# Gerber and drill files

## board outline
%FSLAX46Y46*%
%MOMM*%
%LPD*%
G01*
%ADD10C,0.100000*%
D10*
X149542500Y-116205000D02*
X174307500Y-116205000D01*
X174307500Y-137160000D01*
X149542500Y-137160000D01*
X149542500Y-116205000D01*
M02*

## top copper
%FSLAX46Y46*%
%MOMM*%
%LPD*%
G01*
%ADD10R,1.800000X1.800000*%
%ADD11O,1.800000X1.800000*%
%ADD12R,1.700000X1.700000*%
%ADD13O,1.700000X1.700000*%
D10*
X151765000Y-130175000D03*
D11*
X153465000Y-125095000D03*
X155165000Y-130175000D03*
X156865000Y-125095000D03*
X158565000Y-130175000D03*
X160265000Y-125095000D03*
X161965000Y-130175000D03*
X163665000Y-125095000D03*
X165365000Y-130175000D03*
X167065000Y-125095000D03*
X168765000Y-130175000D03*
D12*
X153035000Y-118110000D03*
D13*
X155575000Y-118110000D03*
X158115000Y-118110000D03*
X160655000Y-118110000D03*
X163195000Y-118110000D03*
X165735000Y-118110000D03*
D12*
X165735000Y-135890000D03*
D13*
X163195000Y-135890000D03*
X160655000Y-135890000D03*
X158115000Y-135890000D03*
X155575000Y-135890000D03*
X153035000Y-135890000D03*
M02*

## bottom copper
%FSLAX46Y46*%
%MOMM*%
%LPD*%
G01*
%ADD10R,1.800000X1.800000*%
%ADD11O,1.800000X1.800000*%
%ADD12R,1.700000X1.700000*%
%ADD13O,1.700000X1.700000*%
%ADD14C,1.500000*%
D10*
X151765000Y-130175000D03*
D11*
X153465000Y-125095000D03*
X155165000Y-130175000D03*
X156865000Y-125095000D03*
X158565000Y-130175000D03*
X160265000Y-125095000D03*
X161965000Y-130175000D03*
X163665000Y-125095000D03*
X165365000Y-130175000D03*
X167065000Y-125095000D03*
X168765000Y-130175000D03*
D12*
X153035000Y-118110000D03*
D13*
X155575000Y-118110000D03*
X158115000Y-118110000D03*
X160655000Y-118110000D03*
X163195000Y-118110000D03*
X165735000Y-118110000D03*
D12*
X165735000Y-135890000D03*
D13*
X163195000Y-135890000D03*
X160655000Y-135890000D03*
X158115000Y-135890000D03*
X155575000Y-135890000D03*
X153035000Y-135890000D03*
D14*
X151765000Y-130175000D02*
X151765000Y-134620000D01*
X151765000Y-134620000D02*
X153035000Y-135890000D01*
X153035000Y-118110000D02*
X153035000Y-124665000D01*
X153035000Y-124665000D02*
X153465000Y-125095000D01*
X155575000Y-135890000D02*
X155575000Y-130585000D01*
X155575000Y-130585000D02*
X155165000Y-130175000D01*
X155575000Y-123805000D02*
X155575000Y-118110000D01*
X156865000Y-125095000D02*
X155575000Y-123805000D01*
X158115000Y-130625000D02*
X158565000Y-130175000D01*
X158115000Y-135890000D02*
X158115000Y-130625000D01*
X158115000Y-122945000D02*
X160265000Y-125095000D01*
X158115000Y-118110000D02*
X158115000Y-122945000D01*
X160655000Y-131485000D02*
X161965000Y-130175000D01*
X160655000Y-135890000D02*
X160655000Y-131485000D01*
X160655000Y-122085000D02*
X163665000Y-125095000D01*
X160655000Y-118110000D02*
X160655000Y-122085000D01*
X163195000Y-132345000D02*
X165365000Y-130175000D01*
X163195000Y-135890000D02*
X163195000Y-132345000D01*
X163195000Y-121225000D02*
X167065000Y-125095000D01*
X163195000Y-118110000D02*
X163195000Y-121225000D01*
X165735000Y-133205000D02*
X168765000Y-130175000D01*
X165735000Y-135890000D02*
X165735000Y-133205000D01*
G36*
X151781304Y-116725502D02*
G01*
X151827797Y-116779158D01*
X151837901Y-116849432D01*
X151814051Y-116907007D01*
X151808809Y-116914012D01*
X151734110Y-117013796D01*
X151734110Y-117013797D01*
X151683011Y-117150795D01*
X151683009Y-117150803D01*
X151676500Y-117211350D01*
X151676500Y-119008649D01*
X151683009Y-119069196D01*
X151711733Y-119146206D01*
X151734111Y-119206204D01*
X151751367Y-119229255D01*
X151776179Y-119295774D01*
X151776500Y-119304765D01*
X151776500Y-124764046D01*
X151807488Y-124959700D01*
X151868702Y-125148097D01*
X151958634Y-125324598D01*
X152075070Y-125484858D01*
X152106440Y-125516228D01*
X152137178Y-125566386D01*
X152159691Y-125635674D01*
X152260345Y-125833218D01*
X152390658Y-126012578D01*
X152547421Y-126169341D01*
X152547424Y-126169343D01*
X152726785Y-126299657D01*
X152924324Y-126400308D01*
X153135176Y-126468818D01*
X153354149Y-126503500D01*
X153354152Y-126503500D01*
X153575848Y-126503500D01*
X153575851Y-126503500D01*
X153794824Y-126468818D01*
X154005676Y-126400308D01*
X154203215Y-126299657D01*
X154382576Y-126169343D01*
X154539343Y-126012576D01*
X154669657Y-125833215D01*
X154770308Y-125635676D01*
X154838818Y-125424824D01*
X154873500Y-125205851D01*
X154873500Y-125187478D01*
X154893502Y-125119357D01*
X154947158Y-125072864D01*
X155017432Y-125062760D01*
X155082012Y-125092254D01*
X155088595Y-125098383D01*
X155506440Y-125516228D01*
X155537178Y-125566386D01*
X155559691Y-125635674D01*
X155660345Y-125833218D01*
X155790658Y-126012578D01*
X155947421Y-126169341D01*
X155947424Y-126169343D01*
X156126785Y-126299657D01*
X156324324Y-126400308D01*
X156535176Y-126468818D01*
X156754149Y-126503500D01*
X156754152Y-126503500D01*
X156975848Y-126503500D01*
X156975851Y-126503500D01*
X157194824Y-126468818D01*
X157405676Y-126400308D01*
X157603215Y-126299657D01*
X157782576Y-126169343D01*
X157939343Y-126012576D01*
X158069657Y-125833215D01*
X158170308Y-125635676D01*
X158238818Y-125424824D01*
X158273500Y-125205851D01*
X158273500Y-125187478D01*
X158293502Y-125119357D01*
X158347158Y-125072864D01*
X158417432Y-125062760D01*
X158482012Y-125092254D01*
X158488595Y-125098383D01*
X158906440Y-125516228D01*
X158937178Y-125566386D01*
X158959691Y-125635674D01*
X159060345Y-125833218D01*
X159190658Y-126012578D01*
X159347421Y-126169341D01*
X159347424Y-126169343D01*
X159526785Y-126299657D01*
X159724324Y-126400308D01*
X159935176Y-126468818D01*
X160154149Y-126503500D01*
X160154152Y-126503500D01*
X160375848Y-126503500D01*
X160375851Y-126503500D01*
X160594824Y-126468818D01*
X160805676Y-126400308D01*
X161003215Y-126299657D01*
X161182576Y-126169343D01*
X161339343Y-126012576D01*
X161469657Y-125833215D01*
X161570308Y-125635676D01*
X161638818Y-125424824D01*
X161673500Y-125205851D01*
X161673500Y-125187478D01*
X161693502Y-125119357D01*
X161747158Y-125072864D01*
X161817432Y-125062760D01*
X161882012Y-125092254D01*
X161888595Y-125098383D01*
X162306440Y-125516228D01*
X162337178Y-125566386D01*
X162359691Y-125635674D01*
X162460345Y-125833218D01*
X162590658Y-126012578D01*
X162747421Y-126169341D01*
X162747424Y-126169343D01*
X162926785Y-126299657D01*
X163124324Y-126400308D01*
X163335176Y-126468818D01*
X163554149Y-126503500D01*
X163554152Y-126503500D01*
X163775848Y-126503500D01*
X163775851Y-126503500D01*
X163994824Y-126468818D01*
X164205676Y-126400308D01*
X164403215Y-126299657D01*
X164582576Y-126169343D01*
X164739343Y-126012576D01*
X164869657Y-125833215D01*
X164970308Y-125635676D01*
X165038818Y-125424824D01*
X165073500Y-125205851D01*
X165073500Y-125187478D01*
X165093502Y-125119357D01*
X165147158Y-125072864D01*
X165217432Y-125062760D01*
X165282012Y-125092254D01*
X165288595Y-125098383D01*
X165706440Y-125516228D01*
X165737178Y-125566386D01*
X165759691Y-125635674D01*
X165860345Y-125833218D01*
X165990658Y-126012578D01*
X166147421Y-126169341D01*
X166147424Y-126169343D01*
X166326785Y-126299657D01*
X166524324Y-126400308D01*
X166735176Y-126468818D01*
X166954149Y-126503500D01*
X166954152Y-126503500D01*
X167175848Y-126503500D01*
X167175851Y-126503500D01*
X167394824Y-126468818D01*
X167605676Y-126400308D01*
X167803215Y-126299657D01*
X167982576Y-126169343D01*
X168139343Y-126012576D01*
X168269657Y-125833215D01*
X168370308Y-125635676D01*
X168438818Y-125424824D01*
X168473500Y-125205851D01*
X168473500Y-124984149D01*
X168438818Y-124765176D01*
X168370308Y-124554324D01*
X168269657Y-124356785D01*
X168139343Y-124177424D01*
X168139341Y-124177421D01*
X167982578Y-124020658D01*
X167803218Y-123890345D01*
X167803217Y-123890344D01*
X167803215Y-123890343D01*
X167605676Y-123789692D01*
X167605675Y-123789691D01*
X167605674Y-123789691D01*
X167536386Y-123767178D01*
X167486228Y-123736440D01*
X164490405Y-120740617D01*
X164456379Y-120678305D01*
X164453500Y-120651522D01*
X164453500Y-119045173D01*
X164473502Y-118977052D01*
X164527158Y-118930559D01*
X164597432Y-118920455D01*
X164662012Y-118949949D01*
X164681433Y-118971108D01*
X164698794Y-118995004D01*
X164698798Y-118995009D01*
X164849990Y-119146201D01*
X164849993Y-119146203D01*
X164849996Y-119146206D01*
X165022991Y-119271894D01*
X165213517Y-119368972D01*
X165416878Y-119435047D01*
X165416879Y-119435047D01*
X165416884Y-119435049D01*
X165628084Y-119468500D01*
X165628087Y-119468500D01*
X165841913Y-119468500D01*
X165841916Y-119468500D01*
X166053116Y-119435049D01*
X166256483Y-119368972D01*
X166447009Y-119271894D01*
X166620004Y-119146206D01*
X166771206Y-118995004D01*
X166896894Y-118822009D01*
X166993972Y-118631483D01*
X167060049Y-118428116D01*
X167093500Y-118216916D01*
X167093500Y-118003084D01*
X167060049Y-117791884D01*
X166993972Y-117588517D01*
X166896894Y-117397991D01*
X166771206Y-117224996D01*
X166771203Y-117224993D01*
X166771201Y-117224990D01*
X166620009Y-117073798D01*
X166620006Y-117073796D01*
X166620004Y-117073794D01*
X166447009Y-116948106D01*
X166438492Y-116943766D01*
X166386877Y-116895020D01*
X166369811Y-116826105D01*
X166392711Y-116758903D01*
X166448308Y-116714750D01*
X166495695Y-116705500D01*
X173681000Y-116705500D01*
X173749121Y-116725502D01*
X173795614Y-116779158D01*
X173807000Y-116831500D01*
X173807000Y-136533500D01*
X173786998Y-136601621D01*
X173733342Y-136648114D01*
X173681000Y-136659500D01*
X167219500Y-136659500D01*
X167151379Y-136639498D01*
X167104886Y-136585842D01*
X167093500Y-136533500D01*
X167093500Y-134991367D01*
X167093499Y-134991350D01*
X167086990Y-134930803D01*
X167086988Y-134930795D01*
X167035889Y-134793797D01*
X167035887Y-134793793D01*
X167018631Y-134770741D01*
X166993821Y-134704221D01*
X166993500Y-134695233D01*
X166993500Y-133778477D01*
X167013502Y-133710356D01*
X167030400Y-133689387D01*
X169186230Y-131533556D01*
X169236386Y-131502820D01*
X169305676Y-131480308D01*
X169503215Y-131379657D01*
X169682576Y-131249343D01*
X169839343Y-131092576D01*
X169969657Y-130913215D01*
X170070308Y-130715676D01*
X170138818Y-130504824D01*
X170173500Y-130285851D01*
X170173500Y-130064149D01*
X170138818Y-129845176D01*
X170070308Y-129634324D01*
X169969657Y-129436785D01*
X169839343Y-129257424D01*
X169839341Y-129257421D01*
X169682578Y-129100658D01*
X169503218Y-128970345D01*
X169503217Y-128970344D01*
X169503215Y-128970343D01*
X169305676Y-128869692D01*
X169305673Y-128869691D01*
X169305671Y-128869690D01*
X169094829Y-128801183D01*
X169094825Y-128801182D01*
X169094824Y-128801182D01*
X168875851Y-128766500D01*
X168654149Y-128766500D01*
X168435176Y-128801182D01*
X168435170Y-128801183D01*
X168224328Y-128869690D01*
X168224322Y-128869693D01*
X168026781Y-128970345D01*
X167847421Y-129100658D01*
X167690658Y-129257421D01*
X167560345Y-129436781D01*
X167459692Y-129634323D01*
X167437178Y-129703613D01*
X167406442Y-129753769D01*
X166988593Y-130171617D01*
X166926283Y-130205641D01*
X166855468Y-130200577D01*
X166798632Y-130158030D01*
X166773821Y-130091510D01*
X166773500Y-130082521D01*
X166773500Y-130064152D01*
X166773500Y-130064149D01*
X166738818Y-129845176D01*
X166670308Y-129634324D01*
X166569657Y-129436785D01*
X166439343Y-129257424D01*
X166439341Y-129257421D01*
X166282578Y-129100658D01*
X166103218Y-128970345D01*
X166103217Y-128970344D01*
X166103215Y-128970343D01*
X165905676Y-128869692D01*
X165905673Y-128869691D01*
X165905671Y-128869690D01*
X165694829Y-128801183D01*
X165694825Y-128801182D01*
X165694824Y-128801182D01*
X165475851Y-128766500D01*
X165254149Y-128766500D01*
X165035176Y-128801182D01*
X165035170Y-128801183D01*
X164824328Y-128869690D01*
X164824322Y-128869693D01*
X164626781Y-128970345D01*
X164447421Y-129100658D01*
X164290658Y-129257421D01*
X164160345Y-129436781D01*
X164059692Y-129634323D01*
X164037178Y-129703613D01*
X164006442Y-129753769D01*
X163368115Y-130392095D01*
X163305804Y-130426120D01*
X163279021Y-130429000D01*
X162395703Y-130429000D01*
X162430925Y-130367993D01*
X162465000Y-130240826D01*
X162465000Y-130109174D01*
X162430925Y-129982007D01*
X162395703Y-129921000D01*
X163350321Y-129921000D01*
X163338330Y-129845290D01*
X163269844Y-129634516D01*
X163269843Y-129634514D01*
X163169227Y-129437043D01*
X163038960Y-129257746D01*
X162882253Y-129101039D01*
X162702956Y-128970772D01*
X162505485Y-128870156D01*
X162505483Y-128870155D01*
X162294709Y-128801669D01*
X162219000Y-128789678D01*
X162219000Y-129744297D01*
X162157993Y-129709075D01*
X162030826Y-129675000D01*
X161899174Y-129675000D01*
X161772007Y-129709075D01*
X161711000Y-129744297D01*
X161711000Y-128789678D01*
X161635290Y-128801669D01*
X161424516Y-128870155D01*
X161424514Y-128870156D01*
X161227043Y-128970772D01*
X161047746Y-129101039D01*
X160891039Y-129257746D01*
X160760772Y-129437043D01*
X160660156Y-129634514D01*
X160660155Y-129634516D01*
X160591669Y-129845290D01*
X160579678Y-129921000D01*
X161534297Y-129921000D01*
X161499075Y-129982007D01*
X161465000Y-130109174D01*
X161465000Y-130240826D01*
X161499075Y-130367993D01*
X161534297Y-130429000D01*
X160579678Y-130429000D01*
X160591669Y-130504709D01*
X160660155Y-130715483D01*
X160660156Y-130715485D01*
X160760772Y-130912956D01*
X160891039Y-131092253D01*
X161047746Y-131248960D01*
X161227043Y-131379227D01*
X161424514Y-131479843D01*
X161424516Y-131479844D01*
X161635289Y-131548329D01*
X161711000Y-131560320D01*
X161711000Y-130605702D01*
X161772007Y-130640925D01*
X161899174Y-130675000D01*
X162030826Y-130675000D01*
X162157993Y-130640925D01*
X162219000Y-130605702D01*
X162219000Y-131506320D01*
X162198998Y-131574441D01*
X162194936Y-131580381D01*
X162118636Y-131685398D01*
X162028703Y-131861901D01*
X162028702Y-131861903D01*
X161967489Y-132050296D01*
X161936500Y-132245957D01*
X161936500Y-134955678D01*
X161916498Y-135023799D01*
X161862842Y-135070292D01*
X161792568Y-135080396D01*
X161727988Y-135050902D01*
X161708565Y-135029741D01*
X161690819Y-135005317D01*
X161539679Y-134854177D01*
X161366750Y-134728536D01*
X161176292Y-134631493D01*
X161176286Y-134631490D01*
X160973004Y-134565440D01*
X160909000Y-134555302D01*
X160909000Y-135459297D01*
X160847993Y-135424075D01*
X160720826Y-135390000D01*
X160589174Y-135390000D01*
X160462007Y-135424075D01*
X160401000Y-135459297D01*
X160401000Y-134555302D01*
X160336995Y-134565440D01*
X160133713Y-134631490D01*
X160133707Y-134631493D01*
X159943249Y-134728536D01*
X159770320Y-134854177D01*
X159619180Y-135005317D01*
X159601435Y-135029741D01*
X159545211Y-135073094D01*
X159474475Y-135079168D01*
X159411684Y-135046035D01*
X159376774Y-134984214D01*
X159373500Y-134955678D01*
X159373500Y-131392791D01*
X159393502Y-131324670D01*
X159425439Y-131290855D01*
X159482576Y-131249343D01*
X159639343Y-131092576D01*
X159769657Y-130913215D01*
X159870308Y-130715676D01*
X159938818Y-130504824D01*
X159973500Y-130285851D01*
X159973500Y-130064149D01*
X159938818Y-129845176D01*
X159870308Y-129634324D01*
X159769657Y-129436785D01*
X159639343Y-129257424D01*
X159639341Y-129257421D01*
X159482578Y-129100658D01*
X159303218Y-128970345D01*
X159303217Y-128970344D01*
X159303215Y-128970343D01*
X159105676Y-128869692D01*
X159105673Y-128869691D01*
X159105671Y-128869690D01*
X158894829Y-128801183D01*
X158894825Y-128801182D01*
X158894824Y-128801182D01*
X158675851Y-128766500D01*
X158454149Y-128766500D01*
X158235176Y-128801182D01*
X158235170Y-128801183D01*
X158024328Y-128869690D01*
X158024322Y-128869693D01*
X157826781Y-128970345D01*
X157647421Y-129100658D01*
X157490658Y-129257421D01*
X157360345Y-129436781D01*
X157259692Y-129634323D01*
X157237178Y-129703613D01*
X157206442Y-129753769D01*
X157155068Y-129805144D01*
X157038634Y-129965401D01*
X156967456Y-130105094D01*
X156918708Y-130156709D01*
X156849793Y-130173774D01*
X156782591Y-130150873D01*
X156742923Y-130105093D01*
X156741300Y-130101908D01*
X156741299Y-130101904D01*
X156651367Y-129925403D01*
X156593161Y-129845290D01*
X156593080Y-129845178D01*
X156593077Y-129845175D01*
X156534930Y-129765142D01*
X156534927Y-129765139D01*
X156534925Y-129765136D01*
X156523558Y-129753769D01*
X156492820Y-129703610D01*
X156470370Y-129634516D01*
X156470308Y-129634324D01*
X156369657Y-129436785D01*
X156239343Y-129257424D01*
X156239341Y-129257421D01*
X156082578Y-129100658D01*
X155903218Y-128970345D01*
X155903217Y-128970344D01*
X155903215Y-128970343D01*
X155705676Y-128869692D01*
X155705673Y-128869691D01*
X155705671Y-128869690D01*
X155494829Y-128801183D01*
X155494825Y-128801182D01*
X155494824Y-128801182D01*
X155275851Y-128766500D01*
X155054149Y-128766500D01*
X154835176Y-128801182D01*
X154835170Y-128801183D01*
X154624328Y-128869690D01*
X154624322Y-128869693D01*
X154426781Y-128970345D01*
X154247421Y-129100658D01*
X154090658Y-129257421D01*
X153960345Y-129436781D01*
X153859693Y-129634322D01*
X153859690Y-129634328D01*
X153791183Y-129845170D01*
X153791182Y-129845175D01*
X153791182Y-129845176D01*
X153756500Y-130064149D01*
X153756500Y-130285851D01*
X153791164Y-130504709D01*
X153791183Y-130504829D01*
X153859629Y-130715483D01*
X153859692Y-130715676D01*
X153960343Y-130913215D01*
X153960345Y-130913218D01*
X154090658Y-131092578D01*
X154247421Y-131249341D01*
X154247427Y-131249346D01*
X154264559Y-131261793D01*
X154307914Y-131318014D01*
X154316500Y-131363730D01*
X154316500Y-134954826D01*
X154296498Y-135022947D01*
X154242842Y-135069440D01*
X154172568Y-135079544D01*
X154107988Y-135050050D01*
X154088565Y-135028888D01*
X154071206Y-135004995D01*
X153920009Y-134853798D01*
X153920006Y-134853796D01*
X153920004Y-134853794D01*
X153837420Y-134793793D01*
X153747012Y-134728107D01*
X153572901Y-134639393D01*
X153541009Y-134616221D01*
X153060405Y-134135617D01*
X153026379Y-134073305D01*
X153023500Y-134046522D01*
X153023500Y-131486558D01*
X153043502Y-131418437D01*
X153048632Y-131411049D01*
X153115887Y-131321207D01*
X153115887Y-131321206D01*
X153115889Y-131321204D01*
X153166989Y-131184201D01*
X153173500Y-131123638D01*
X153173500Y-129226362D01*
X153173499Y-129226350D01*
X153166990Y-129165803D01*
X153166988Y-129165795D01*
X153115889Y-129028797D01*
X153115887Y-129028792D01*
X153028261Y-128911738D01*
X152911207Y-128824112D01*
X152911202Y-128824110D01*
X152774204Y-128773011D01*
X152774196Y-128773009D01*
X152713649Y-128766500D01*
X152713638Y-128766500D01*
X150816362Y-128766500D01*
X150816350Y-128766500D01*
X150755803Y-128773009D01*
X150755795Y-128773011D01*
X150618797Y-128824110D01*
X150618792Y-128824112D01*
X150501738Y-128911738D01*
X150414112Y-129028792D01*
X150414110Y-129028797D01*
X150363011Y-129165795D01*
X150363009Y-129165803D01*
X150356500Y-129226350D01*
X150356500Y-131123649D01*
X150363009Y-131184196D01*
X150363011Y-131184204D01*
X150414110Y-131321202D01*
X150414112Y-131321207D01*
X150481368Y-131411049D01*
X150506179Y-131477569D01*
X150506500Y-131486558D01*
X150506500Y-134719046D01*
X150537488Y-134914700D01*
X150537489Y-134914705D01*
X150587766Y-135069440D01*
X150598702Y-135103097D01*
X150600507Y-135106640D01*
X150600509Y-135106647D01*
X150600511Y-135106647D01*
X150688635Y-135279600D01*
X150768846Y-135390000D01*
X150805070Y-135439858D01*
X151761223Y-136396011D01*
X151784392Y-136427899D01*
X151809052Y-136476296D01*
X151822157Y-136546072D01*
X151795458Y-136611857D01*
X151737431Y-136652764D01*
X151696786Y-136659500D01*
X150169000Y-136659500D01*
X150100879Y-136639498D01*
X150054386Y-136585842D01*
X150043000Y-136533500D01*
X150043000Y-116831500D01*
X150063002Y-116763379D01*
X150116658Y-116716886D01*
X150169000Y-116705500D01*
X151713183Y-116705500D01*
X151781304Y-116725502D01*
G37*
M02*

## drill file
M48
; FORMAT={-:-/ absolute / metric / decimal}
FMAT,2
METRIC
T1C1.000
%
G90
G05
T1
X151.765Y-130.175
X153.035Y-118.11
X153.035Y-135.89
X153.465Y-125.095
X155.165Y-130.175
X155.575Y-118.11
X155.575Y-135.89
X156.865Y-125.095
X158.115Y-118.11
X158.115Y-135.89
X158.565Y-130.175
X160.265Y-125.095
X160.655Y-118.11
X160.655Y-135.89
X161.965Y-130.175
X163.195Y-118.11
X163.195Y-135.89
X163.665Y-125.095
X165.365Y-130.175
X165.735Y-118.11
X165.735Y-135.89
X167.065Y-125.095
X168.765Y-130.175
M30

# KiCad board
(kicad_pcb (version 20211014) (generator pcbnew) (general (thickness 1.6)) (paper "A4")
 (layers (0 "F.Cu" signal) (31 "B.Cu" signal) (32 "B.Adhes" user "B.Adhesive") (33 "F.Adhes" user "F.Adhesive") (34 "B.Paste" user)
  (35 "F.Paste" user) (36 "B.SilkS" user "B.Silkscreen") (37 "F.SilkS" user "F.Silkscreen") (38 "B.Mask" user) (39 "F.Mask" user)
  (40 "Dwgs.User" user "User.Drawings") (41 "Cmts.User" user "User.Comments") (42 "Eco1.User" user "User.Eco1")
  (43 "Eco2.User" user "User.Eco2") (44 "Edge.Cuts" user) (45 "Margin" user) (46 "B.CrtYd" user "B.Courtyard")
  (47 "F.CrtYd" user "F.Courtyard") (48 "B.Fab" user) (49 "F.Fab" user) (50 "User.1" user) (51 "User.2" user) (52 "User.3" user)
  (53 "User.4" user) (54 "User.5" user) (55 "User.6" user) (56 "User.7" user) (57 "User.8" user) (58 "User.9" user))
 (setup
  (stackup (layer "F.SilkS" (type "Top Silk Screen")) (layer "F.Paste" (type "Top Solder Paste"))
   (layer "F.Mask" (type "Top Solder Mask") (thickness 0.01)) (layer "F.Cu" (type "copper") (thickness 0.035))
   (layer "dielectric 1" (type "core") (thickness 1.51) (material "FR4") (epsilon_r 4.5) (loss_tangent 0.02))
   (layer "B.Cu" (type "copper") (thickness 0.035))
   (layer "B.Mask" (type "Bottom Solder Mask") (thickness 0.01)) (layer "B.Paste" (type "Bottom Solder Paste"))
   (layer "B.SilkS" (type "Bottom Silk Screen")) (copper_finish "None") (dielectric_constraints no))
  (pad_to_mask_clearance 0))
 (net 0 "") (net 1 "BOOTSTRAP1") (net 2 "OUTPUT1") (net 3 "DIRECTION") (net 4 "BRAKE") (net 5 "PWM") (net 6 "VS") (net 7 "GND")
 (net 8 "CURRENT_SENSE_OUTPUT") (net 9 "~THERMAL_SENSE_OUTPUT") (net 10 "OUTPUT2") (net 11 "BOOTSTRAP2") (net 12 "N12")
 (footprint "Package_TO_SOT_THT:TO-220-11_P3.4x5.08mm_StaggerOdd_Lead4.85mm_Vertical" (layer "F.Cu") (at 151.765 130.175)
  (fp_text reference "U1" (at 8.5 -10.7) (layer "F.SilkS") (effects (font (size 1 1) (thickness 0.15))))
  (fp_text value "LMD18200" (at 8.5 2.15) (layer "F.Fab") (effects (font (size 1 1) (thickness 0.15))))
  (pad "1" thru_hole rect (at 0 0) (size 1.8 1.8) (drill 1) (layers *.Cu *.Mask) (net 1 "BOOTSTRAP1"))
  (pad "2" thru_hole oval (at 1.7 -5.08) (size 1.8 1.8) (drill 1) (layers *.Cu *.Mask) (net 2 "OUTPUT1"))
  (pad "3" thru_hole oval (at 3.4 0) (size 1.8 1.8) (drill 1) (layers *.Cu *.Mask) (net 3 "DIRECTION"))
  (pad "4" thru_hole oval (at 5.1 -5.08) (size 1.8 1.8) (drill 1) (layers *.Cu *.Mask) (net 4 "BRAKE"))
  (pad "5" thru_hole oval (at 6.8 0) (size 1.8 1.8) (drill 1) (layers *.Cu *.Mask) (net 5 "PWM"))
  (pad "6" thru_hole oval (at 8.5 -5.08) (size 1.8 1.8) (drill 1) (layers *.Cu *.Mask) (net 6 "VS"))
  (pad "7" thru_hole oval (at 10.2 0) (size 1.8 1.8) (drill 1) (layers *.Cu *.Mask) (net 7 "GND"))
  (pad "8" thru_hole oval (at 11.9 -5.08) (size 1.8 1.8) (drill 1) (layers *.Cu *.Mask) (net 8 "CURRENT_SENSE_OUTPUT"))
  (pad "9" thru_hole oval (at 13.6 0) (size 1.8 1.8) (drill 1) (layers *.Cu *.Mask) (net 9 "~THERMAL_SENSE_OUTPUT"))
  (pad "10" thru_hole oval (at 15.3 -5.08) (size 1.8 1.8) (drill 1) (layers *.Cu *.Mask) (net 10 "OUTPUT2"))
  (pad "11" thru_hole oval (at 17 0) (size 1.8 1.8) (drill 1) (layers *.Cu *.Mask) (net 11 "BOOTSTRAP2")))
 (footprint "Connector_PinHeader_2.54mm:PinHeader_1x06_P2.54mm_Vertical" (layer "F.Cu") (at 153.035 118.11 90)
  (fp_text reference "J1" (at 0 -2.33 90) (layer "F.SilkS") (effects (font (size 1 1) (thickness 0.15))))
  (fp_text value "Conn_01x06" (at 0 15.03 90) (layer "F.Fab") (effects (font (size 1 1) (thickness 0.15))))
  (pad "1" thru_hole rect (at 0 0 90) (size 1.7 1.7) (drill 1) (layers *.Cu *.Mask) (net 2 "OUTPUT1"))
  (pad "2" thru_hole oval (at 0 2.54 90) (size 1.7 1.7) (drill 1) (layers *.Cu *.Mask) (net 4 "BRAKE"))
  (pad "3" thru_hole oval (at 0 5.08 90) (size 1.7 1.7) (drill 1) (layers *.Cu *.Mask) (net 6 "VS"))
  (pad "4" thru_hole oval (at 0 7.62 90) (size 1.7 1.7) (drill 1) (layers *.Cu *.Mask) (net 8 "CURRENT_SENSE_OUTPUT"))
  (pad "5" thru_hole oval (at 0 10.16 90) (size 1.7 1.7) (drill 1) (layers *.Cu *.Mask) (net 10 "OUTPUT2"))
  (pad "6" thru_hole oval (at 0 12.7 90) (size 1.7 1.7) (drill 1) (layers *.Cu *.Mask) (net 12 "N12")))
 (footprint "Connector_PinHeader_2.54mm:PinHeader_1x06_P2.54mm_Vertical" (layer "F.Cu") (at 165.735 135.89 -90)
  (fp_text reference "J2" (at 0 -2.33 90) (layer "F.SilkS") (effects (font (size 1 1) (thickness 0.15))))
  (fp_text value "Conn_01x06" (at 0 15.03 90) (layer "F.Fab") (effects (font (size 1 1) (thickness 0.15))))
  (pad "1" thru_hole rect (at 0 0 270) (size 1.7 1.7) (drill 1) (layers *.Cu *.Mask) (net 11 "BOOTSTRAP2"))
  (pad "2" thru_hole oval (at 0 2.54 270) (size 1.7 1.7) (drill 1) (layers *.Cu *.Mask) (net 9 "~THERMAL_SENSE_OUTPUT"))
  (pad "3" thru_hole oval (at 0 5.08 270) (size 1.7 1.7) (drill 1) (layers *.Cu *.Mask) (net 7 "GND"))
  (pad "4" thru_hole oval (at 0 7.62 270) (size 1.7 1.7) (drill 1) (layers *.Cu *.Mask) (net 5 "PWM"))
  (pad "5" thru_hole oval (at 0 10.16 270) (size 1.7 1.7) (drill 1) (layers *.Cu *.Mask) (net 3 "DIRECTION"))
  (pad "6" thru_hole oval (at 0 12.7 270) (size 1.7 1.7) (drill 1) (layers *.Cu *.Mask) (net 1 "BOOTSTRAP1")))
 (gr_rect (start 149.5425 116.205) (end 174.3075 137.16) (layer "Edge.Cuts") (width 0.1) (fill none))
 (segment (start 151.765 130.175) (end 151.765 134.62) (width 1.5) (layer "B.Cu") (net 1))
 (segment (start 151.765 134.62) (end 153.035 135.89) (width 1.5) (layer "B.Cu") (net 1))
 (segment (start 153.035 118.11) (end 153.035 124.665) (width 1.5) (layer "B.Cu") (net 2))
 (segment (start 153.035 124.665) (end 153.465 125.095) (width 1.5) (layer "B.Cu") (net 2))
 (segment (start 155.575 135.89) (end 155.575 130.585) (width 1.5) (layer "B.Cu") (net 3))
 (segment (start 155.575 130.585) (end 155.165 130.175) (width 1.5) (layer "B.Cu") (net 3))
 (segment (start 155.575 123.805) (end 155.575 118.11) (width 1.5) (layer "B.Cu") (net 4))
 (segment (start 156.865 125.095) (end 155.575 123.805) (width 1.5) (layer "B.Cu") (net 4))
 (segment (start 158.115 130.625) (end 158.565 130.175) (width 1.5) (layer "B.Cu") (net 5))
 (segment (start 158.115 135.89) (end 158.115 130.625) (width 1.5) (layer "B.Cu") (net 5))
 (segment (start 158.115 122.945) (end 160.265 125.095) (width 1.5) (layer "B.Cu") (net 6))
 (segment (start 158.115 118.11) (end 158.115 122.945) (width 1.5) (layer "B.Cu") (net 6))
 (segment (start 160.655 131.485) (end 161.965 130.175) (width 1.5) (layer "B.Cu") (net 7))
 (segment (start 160.655 135.89) (end 160.655 131.485) (width 1.5) (layer "B.Cu") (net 7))
 (segment (start 160.655 122.085) (end 163.665 125.095) (width 1.5) (layer "B.Cu") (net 8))
 (segment (start 160.655 118.11) (end 160.655 122.085) (width 1.5) (layer "B.Cu") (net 8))
 (segment (start 163.195 132.345) (end 165.365 130.175) (width 1.5) (layer "B.Cu") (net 9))
 (segment (start 163.195 135.89) (end 163.195 132.345) (width 1.5) (layer "B.Cu") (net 9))
 (segment (start 163.195 121.225) (end 167.065 125.095) (width 1.5) (layer "B.Cu") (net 10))
 (segment (start 163.195 118.11) (end 163.195 121.225) (width 1.5) (layer "B.Cu") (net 10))
 (segment (start 165.735 133.205) (end 168.765 130.175) (width 1.5) (layer "B.Cu") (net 11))
 (segment (start 165.735 135.89) (end 165.735 133.205) (width 1.5) (layer "B.Cu") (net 11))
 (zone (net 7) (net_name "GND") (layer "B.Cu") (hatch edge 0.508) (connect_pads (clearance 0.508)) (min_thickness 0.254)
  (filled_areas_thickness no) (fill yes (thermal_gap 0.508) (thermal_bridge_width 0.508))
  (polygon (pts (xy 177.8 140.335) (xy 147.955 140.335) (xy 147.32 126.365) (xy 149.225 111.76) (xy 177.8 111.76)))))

